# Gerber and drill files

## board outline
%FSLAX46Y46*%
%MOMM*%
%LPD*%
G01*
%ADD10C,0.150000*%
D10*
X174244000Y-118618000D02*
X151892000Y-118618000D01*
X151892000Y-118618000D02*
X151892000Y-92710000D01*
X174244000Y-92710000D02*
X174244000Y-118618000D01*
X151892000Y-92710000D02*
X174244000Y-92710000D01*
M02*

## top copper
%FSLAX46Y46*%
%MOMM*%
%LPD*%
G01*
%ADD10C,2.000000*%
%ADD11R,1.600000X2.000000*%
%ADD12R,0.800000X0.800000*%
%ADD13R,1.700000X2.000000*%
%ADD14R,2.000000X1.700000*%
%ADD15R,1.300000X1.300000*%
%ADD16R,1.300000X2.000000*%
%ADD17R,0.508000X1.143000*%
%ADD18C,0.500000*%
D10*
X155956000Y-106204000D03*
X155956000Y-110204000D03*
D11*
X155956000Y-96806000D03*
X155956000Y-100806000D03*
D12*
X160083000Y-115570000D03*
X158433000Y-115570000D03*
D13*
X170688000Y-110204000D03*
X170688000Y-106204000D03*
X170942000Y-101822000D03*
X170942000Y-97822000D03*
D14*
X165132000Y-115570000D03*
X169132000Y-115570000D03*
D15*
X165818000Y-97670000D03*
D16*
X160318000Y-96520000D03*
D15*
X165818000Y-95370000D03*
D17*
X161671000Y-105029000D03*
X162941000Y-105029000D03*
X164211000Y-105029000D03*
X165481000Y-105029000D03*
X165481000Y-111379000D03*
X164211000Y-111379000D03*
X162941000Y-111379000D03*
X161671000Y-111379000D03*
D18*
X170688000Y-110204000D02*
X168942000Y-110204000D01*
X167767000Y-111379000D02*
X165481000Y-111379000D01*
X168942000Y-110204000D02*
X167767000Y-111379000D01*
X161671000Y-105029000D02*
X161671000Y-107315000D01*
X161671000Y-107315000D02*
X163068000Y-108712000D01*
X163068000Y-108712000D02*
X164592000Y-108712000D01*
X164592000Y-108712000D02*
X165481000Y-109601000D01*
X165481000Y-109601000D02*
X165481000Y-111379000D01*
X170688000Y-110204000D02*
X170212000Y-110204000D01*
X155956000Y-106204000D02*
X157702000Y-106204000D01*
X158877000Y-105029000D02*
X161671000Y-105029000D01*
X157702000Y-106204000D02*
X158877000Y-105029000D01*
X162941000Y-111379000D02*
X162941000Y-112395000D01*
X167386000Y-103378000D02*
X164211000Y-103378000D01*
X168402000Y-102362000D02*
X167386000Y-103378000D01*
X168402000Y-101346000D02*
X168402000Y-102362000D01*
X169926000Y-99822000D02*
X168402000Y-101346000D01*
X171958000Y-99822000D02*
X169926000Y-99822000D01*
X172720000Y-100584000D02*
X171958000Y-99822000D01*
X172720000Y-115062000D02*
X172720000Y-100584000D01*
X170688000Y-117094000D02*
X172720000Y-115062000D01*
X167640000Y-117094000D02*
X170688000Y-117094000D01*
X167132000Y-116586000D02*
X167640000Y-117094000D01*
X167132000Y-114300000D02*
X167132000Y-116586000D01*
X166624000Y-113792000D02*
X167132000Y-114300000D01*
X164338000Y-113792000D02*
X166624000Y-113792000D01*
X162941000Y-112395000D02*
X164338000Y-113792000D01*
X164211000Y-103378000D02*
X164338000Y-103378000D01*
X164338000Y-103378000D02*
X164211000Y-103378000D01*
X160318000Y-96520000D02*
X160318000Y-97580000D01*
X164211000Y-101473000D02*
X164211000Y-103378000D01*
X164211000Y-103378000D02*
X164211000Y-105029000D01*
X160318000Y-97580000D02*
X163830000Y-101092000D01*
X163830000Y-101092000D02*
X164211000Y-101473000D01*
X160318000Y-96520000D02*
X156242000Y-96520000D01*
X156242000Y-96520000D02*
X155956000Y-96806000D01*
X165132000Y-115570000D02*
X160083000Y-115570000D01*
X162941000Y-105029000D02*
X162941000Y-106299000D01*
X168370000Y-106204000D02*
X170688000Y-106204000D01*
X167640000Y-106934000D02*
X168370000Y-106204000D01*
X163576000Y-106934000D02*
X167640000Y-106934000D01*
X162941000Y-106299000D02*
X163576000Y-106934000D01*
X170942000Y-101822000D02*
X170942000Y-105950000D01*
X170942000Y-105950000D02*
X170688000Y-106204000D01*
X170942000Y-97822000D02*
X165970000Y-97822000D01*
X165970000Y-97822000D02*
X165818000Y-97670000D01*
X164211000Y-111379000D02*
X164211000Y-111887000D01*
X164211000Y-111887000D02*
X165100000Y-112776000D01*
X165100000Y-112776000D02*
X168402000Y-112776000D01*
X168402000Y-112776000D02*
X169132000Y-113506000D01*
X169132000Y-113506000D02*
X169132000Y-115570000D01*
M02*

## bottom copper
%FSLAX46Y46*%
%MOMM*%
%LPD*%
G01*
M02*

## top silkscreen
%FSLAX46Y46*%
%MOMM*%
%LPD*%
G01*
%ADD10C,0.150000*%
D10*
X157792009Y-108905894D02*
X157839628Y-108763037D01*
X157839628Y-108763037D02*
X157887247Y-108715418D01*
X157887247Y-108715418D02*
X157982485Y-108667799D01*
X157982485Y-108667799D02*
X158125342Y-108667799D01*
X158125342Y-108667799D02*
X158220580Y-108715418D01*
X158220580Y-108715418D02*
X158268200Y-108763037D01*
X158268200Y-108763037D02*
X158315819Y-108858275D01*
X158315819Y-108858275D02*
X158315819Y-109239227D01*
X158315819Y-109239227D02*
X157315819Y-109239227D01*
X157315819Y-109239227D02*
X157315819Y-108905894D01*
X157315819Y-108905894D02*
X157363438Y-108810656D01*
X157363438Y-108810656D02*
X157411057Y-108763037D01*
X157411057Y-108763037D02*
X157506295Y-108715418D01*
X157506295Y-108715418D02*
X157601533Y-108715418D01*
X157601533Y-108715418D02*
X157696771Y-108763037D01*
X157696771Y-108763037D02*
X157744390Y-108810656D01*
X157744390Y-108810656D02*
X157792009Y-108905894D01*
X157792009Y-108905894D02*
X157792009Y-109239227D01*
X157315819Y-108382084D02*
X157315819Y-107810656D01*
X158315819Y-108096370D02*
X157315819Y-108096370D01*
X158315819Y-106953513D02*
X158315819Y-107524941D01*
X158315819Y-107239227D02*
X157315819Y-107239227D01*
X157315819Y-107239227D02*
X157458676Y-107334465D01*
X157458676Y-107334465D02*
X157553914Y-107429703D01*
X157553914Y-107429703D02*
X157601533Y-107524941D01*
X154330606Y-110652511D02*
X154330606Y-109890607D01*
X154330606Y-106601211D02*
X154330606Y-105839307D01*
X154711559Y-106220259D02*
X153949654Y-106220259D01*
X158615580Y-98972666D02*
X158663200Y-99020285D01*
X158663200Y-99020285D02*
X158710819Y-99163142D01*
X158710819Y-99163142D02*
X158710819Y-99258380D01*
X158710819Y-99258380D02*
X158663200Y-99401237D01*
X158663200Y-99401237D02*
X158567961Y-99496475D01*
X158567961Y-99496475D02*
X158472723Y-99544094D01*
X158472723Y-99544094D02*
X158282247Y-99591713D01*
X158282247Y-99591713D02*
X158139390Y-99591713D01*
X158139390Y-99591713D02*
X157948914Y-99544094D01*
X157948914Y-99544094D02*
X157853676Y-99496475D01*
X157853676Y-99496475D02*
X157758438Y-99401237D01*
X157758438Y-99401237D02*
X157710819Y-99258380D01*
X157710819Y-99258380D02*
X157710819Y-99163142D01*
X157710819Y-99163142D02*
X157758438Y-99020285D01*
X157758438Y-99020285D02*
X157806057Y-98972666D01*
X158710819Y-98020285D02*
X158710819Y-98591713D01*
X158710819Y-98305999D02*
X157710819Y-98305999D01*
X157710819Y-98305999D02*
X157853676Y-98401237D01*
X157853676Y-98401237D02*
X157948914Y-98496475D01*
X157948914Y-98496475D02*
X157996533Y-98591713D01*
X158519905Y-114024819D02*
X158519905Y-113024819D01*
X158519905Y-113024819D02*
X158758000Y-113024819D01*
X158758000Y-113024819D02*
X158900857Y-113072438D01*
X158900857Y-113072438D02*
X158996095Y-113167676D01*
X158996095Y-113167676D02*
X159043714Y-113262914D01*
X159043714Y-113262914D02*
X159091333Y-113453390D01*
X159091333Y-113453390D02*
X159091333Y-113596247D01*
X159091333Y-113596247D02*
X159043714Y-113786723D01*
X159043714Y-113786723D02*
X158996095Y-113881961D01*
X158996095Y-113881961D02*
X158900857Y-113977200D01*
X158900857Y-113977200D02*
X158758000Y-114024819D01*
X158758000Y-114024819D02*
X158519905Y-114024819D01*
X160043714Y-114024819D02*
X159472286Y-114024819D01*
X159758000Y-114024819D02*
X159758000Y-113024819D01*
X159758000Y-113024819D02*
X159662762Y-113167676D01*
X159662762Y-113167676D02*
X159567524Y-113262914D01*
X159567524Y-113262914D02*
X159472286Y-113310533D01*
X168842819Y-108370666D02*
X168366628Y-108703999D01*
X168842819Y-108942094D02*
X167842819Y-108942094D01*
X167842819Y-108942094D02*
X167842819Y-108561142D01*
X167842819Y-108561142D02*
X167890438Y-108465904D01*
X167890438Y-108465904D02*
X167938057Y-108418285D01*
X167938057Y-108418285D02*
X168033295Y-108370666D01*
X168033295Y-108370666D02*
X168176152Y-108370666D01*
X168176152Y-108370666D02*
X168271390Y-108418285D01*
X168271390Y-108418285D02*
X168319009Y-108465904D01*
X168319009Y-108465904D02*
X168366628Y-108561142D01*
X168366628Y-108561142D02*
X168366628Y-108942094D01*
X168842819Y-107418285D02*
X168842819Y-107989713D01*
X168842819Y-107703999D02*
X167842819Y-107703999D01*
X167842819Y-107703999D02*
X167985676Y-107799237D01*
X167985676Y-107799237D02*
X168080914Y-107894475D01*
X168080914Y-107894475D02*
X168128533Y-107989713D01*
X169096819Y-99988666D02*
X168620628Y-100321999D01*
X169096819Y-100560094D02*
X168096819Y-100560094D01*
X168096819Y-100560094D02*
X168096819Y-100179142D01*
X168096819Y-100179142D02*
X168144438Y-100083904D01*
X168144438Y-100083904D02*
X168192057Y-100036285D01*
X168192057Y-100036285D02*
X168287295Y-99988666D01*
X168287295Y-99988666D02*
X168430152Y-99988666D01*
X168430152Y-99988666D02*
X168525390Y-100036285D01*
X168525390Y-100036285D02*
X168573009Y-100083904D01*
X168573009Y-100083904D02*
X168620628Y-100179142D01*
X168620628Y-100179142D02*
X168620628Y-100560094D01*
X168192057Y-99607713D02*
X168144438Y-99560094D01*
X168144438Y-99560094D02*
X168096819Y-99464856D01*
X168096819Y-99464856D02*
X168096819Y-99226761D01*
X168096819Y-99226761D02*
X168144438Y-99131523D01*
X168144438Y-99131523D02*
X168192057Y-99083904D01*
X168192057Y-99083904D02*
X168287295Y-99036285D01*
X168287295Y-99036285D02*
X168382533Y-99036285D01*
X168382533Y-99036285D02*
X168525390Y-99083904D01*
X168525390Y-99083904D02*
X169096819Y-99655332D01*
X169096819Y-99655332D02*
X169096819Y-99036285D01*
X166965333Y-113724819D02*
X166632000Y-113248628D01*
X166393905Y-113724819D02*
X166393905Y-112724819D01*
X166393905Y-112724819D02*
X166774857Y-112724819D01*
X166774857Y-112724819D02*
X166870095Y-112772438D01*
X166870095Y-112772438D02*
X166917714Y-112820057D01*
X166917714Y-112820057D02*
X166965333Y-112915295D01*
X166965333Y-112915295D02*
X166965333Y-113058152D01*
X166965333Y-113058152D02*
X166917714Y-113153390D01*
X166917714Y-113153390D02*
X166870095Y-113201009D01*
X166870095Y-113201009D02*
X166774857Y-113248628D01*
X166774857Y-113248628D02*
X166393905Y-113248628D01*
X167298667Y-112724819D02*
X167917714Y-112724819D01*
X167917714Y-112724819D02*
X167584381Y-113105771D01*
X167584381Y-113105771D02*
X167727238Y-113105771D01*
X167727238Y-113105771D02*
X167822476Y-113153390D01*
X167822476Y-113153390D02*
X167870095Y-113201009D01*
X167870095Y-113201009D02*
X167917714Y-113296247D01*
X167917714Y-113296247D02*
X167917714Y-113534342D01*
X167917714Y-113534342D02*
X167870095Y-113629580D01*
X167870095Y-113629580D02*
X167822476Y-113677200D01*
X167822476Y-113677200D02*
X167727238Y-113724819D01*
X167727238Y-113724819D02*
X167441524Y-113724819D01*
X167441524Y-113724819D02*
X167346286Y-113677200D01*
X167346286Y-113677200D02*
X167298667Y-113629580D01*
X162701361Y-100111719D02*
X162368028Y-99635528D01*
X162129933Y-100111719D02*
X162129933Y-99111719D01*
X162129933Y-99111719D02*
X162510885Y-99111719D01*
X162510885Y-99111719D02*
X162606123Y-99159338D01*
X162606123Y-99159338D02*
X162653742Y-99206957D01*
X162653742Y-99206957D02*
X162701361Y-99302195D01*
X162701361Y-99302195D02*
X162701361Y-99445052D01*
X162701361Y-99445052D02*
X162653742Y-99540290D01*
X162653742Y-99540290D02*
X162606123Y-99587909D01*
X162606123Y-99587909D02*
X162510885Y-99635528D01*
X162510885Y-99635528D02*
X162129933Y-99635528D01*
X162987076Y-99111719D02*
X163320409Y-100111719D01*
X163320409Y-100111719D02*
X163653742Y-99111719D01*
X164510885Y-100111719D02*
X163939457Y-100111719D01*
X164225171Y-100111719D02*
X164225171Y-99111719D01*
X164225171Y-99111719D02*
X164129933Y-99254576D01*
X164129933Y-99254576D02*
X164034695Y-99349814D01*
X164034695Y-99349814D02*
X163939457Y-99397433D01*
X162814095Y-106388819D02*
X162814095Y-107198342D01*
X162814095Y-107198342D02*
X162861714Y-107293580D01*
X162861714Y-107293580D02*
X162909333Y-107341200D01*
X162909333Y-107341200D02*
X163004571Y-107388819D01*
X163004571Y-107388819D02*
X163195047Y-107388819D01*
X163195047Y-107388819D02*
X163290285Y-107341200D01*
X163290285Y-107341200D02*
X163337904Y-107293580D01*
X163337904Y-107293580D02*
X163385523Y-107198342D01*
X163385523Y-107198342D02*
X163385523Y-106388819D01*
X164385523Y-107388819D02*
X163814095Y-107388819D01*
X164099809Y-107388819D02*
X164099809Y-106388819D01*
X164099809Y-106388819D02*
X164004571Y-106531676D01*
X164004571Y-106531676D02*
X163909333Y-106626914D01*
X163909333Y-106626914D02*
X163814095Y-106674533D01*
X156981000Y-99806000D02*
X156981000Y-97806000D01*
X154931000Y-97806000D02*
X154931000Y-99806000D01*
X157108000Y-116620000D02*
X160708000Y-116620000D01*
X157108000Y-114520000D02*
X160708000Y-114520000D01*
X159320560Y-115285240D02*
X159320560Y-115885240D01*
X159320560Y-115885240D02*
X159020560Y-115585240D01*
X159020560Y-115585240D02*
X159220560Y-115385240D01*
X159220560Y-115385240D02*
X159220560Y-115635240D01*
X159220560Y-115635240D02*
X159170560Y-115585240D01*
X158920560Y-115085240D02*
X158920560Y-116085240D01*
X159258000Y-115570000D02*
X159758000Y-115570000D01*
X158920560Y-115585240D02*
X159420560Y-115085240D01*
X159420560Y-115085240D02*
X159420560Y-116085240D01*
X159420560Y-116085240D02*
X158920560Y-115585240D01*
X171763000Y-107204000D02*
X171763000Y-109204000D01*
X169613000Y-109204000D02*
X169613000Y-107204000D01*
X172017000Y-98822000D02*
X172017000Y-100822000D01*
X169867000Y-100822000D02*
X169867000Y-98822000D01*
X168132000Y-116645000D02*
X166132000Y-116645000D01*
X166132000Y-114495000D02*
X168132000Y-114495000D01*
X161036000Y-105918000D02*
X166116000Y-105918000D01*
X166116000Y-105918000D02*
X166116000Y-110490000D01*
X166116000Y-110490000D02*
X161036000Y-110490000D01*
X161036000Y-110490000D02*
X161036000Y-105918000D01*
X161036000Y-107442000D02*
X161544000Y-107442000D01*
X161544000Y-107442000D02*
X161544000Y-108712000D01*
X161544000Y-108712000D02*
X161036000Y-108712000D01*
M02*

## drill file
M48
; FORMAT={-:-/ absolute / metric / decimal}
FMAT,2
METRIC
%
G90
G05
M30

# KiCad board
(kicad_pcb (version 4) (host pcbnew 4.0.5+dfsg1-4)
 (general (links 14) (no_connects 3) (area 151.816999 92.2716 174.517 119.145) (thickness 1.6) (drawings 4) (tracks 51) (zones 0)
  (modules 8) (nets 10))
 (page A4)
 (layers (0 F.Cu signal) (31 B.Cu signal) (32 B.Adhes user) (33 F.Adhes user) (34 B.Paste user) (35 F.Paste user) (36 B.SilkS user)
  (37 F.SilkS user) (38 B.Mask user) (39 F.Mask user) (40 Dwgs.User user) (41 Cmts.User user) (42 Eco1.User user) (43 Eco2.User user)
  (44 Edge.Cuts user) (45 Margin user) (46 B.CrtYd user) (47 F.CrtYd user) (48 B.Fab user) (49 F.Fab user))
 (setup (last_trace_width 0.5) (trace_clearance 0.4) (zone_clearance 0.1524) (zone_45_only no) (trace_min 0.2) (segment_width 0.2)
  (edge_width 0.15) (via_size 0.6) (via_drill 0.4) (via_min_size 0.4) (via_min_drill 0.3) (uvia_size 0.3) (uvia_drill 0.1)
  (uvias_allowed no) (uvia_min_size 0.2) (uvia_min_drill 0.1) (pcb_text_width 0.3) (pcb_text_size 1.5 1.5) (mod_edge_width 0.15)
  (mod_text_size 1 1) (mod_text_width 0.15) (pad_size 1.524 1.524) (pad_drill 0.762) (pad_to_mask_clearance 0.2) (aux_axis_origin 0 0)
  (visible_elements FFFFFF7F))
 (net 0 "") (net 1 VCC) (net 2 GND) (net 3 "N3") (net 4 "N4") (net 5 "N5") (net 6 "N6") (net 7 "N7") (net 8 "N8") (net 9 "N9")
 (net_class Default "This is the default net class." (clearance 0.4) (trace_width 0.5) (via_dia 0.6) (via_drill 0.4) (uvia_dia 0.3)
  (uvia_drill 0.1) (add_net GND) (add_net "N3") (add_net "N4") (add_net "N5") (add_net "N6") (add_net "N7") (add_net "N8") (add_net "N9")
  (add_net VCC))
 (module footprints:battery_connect (layer F.Cu) (at 155.956 108.204 270)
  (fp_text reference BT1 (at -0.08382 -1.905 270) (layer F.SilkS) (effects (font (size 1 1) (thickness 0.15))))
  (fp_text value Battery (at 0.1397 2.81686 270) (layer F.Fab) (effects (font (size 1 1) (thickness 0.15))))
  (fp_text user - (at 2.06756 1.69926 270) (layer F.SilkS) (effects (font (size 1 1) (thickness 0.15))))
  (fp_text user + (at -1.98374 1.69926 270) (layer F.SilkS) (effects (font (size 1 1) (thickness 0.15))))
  (pad 1 smd circle (at -2 0 270) (size 2 2) (layers F.Cu F.Paste F.Mask) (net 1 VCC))
  (pad 2 smd circle (at 2 0 270) (size 2 2) (layers F.Cu F.Paste F.Mask) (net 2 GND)))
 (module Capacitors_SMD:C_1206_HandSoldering (layer F.Cu) (at 155.956 98.806 270)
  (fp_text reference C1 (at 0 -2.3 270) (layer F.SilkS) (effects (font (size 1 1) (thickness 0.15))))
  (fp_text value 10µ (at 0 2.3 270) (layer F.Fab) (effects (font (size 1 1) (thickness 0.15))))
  (fp_line (start 1 -1.025) (end -1 -1.025) (layer F.SilkS) (width 0.15))
  (fp_line (start -1 1.025) (end 1 1.025) (layer F.SilkS) (width 0.15))
  (pad 1 smd rect (at -2 0 270) (size 2 1.6) (layers F.Cu F.Paste F.Mask) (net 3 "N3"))
  (pad 2 smd rect (at 2 0 270) (size 2 1.6) (layers F.Cu F.Paste F.Mask) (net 2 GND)))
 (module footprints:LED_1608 (layer F.Cu) (at 159.258 115.57)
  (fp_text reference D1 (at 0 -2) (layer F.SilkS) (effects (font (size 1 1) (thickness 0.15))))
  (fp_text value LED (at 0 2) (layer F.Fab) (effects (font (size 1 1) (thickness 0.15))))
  (fp_line (start -2.15 1.05) (end 1.45 1.05) (layer F.SilkS) (width 0.15))
  (fp_line (start -2.15 -1.05) (end 1.45 -1.05) (layer F.SilkS) (width 0.15))
  (fp_line (start 0.06256 -0.28476) (end 0.06256 0.31524) (layer F.SilkS) (width 0.15))
  (fp_line (start 0.06256 0.31524) (end -0.23744 0.01524) (layer F.SilkS) (width 0.15))
  (fp_line (start -0.23744 0.01524) (end -0.03744 -0.18476) (layer F.SilkS) (width 0.15))
  (fp_line (start -0.03744 -0.18476) (end -0.03744 0.06524) (layer F.SilkS) (width 0.15))
  (fp_line (start -0.03744 0.06524) (end -0.08744 0.01524) (layer F.SilkS) (width 0.15))
  (fp_line (start -0.33744 -0.48476) (end -0.33744 0.51524) (layer F.SilkS) (width 0.15))
  (fp_line (start 0 0) (end 0.5 0) (layer F.SilkS) (width 0.15))
  (fp_line (start -0.33744 0.01524) (end 0.16256 -0.48476) (layer F.SilkS) (width 0.15))
  (fp_line (start 0.16256 -0.48476) (end 0.16256 0.51524) (layer F.SilkS) (width 0.15))
  (fp_line (start 0.16256 0.51524) (end -0.33744 0.01524) (layer F.SilkS) (width 0.15))
  (pad 2 smd rect (at 0.825 0 180) (size 0.8 0.8) (layers F.Cu F.Paste F.Mask) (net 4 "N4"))
  (pad 1 smd rect (at -0.825 0 180) (size 0.8 0.8) (layers F.Cu F.Paste F.Mask) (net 2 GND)))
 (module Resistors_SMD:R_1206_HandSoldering (layer F.Cu) (at 170.688 108.204 90)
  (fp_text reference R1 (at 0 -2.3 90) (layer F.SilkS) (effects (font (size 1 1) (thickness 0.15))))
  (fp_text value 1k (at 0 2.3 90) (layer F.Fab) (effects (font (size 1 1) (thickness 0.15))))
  (fp_line (start 1 1.075) (end -1 1.075) (layer F.SilkS) (width 0.15))
  (fp_line (start -1 -1.075) (end 1 -1.075) (layer F.SilkS) (width 0.15))
  (pad 1 smd rect (at -2 0 90) (size 2 1.7) (layers F.Cu F.Paste F.Mask) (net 1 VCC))
  (pad 2 smd rect (at 2 0 90) (size 2 1.7) (layers F.Cu F.Paste F.Mask) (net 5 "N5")))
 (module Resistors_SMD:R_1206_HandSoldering (layer F.Cu) (at 170.942 99.822 90)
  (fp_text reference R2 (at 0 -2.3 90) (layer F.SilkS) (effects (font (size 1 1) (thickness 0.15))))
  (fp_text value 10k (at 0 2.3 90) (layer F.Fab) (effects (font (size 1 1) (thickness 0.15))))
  (fp_line (start 1 1.075) (end -1 1.075) (layer F.SilkS) (width 0.15))
  (fp_line (start -1 -1.075) (end 1 -1.075) (layer F.SilkS) (width 0.15))
  (pad 1 smd rect (at -2 0 90) (size 2 1.7) (layers F.Cu F.Paste F.Mask) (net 5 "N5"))
  (pad 2 smd rect (at 2 0 90) (size 2 1.7) (layers F.Cu F.Paste F.Mask) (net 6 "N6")))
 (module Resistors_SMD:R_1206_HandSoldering (layer F.Cu) (at 167.132 115.57)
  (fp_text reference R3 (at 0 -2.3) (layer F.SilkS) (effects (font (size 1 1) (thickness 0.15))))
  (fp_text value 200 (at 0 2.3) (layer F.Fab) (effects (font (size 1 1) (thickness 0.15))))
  (fp_line (start 1 1.075) (end -1 1.075) (layer F.SilkS) (width 0.15))
  (fp_line (start -1 -1.075) (end 1 -1.075) (layer F.SilkS) (width 0.15))
  (pad 1 smd rect (at -2 0) (size 2 1.7) (layers F.Cu F.Paste F.Mask) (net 4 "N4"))
  (pad 2 smd rect (at 2 0) (size 2 1.7) (layers F.Cu F.Paste F.Mask) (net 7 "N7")))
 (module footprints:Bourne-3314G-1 (layer F.Cu) (at 163.068 96.52 270)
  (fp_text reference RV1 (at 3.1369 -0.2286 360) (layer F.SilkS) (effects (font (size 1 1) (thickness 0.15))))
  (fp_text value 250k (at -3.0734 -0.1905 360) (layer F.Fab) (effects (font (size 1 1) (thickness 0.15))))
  (pad 1 smd rect (at 1.15 -2.75 270) (size 1.3 1.3) (layers F.Cu F.Paste F.Mask) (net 6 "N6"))
  (pad 2 smd rect (at 0 2.75 270) (size 2 1.3) (layers F.Cu F.Paste F.Mask) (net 3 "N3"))
  (pad 3 smd rect (at -1.15 -2.75 270) (size 1.3 1.3) (layers F.Cu F.Paste F.Mask) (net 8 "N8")))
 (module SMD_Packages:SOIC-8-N (layer F.Cu) (at 163.576 108.204)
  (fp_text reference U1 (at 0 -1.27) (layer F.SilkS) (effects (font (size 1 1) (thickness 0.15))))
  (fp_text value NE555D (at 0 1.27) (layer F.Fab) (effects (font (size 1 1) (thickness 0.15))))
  (fp_line (start -2.54 -2.286) (end 2.54 -2.286) (layer F.SilkS) (width 0.15))
  (fp_line (start 2.54 -2.286) (end 2.54 2.286) (layer F.SilkS) (width 0.15))
  (fp_line (start 2.54 2.286) (end -2.54 2.286) (layer F.SilkS) (width 0.15))
  (fp_line (start -2.54 2.286) (end -2.54 -2.286) (layer F.SilkS) (width 0.15))
  (fp_line (start -2.54 -0.762) (end -2.032 -0.762) (layer F.SilkS) (width 0.15))
  (fp_line (start -2.032 -0.762) (end -2.032 0.508) (layer F.SilkS) (width 0.15))
  (fp_line (start -2.032 0.508) (end -2.54 0.508) (layer F.SilkS) (width 0.15))
  (pad 8 smd rect (at -1.905 -3.175) (size 0.508 1.143) (layers F.Cu F.Paste F.Mask) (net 1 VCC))
  (pad 7 smd rect (at -0.635 -3.175) (size 0.508 1.143) (layers F.Cu F.Paste F.Mask) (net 5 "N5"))
  (pad 6 smd rect (at 0.635 -3.175) (size 0.508 1.143) (layers F.Cu F.Paste F.Mask) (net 3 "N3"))
  (pad 5 smd rect (at 1.905 -3.175) (size 0.508 1.143) (layers F.Cu F.Paste F.Mask) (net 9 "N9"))
  (pad 4 smd rect (at 1.905 3.175) (size 0.508 1.143) (layers F.Cu F.Paste F.Mask) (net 1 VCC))
  (pad 3 smd rect (at 0.635 3.175) (size 0.508 1.143) (layers F.Cu F.Paste F.Mask) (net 7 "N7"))
  (pad 2 smd rect (at -0.635 3.175) (size 0.508 1.143) (layers F.Cu F.Paste F.Mask) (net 3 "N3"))
  (pad 1 smd rect (at -1.905 3.175) (size 0.508 1.143) (layers F.Cu F.Paste F.Mask) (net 2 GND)))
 (gr_line (start 174.244 118.618) (end 151.892 118.618) (angle 90) (layer Edge.Cuts) (width 0.15))
 (gr_line (start 151.892 118.618) (end 151.892 92.71) (angle 90) (layer Edge.Cuts) (width 0.15))
 (gr_line (start 174.244 92.71) (end 174.244 118.618) (angle 90) (layer Edge.Cuts) (width 0.15))
 (gr_line (start 151.892 92.71) (end 174.244 92.71) (angle 90) (layer Edge.Cuts) (width 0.15))
 (segment (start 170.688 110.204) (end 168.942 110.204) (width 0.5) (layer F.Cu) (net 1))
 (segment (start 167.767 111.379) (end 165.481 111.379) (width 0.5) (layer F.Cu) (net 1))
 (segment (start 168.942 110.204) (end 167.767 111.379) (width 0.5) (layer F.Cu) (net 1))
 (segment (start 161.671 105.029) (end 161.671 107.315) (width 0.5) (layer F.Cu) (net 1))
 (segment (start 161.671 107.315) (end 163.068 108.712) (width 0.5) (layer F.Cu) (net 1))
 (segment (start 163.068 108.712) (end 164.592 108.712) (width 0.5) (layer F.Cu) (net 1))
 (segment (start 164.592 108.712) (end 165.481 109.601) (width 0.5) (layer F.Cu) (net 1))
 (segment (start 165.481 109.601) (end 165.481 111.379) (width 0.5) (layer F.Cu) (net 1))
 (segment (start 170.688 110.204) (end 170.212 110.204) (width 0.5) (layer F.Cu) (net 1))
 (segment (start 155.956 106.204) (end 157.702 106.204) (width 0.5) (layer F.Cu) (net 1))
 (segment (start 158.877 105.029) (end 161.671 105.029) (width 0.5) (layer F.Cu) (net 1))
 (segment (start 157.702 106.204) (end 158.877 105.029) (width 0.5) (layer F.Cu) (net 1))
 (segment (start 162.941 111.379) (end 162.941 112.395) (width 0.5) (layer F.Cu) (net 3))
 (segment (start 167.386 103.378) (end 164.211 103.378) (width 0.5) (layer F.Cu) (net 3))
 (segment (start 168.402 102.362) (end 167.386 103.378) (width 0.5) (layer F.Cu) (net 3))
 (segment (start 168.402 101.346) (end 168.402 102.362) (width 0.5) (layer F.Cu) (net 3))
 (segment (start 169.926 99.822) (end 168.402 101.346) (width 0.5) (layer F.Cu) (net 3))
 (segment (start 171.958 99.822) (end 169.926 99.822) (width 0.5) (layer F.Cu) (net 3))
 (segment (start 172.72 100.584) (end 171.958 99.822) (width 0.5) (layer F.Cu) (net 3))
 (segment (start 172.72 115.062) (end 172.72 100.584) (width 0.5) (layer F.Cu) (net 3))
 (segment (start 170.688 117.094) (end 172.72 115.062) (width 0.5) (layer F.Cu) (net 3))
 (segment (start 167.64 117.094) (end 170.688 117.094) (width 0.5) (layer F.Cu) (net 3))
 (segment (start 167.132 116.586) (end 167.64 117.094) (width 0.5) (layer F.Cu) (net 3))
 (segment (start 167.132 114.3) (end 167.132 116.586) (width 0.5) (layer F.Cu) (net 3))
 (segment (start 166.624 113.792) (end 167.132 114.3) (width 0.5) (layer F.Cu) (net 3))
 (segment (start 164.338 113.792) (end 166.624 113.792) (width 0.5) (layer F.Cu) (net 3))
 (segment (start 162.941 112.395) (end 164.338 113.792) (width 0.5) (layer F.Cu) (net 3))
 (segment (start 164.211 103.378) (end 164.338 103.378) (width 0.5) (layer F.Cu) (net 3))
 (segment (start 164.338 103.378) (end 164.211 103.378) (width 0.5) (layer F.Cu) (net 3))
 (segment (start 160.318 96.52) (end 160.318 97.58) (width 0.5) (layer F.Cu) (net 3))
 (segment (start 164.211 101.473) (end 164.211 103.378) (width 0.5) (layer F.Cu) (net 3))
 (segment (start 164.211 103.378) (end 164.211 105.029) (width 0.5) (layer F.Cu) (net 3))
 (segment (start 160.318 97.58) (end 163.83 101.092) (width 0.5) (layer F.Cu) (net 3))
 (segment (start 163.83 101.092) (end 164.211 101.473) (width 0.5) (layer F.Cu) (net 3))
 (segment (start 160.318 96.52) (end 156.242 96.52) (width 0.5) (layer F.Cu) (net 3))
 (segment (start 156.242 96.52) (end 155.956 96.806) (width 0.5) (layer F.Cu) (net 3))
 (segment (start 165.132 115.57) (end 160.083 115.57) (width 0.5) (layer F.Cu) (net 4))
 (segment (start 162.941 105.029) (end 162.941 106.299) (width 0.5) (layer F.Cu) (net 5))
 (segment (start 168.37 106.204) (end 170.688 106.204) (width 0.5) (layer F.Cu) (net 5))
 (segment (start 167.64 106.934) (end 168.37 106.204) (width 0.5) (layer F.Cu) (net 5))
 (segment (start 163.576 106.934) (end 167.64 106.934) (width 0.5) (layer F.Cu) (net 5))
 (segment (start 162.941 106.299) (end 163.576 106.934) (width 0.5) (layer F.Cu) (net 5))
 (segment (start 170.942 101.822) (end 170.942 105.95) (width 0.5) (layer F.Cu) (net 5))
 (segment (start 170.942 105.95) (end 170.688 106.204) (width 0.5) (layer F.Cu) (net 5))
 (segment (start 170.942 97.822) (end 165.97 97.822) (width 0.5) (layer F.Cu) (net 6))
 (segment (start 165.97 97.822) (end 165.818 97.67) (width 0.5) (layer F.Cu) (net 6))
 (segment (start 164.211 111.379) (end 164.211 111.887) (width 0.5) (layer F.Cu) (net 7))
 (segment (start 164.211 111.887) (end 165.1 112.776) (width 0.5) (layer F.Cu) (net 7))
 (segment (start 165.1 112.776) (end 168.402 112.776) (width 0.5) (layer F.Cu) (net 7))
 (segment (start 168.402 112.776) (end 169.132 113.506) (width 0.5) (layer F.Cu) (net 7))
 (segment (start 169.132 113.506) (end 169.132 115.57) (width 0.5) (layer F.Cu) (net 7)))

